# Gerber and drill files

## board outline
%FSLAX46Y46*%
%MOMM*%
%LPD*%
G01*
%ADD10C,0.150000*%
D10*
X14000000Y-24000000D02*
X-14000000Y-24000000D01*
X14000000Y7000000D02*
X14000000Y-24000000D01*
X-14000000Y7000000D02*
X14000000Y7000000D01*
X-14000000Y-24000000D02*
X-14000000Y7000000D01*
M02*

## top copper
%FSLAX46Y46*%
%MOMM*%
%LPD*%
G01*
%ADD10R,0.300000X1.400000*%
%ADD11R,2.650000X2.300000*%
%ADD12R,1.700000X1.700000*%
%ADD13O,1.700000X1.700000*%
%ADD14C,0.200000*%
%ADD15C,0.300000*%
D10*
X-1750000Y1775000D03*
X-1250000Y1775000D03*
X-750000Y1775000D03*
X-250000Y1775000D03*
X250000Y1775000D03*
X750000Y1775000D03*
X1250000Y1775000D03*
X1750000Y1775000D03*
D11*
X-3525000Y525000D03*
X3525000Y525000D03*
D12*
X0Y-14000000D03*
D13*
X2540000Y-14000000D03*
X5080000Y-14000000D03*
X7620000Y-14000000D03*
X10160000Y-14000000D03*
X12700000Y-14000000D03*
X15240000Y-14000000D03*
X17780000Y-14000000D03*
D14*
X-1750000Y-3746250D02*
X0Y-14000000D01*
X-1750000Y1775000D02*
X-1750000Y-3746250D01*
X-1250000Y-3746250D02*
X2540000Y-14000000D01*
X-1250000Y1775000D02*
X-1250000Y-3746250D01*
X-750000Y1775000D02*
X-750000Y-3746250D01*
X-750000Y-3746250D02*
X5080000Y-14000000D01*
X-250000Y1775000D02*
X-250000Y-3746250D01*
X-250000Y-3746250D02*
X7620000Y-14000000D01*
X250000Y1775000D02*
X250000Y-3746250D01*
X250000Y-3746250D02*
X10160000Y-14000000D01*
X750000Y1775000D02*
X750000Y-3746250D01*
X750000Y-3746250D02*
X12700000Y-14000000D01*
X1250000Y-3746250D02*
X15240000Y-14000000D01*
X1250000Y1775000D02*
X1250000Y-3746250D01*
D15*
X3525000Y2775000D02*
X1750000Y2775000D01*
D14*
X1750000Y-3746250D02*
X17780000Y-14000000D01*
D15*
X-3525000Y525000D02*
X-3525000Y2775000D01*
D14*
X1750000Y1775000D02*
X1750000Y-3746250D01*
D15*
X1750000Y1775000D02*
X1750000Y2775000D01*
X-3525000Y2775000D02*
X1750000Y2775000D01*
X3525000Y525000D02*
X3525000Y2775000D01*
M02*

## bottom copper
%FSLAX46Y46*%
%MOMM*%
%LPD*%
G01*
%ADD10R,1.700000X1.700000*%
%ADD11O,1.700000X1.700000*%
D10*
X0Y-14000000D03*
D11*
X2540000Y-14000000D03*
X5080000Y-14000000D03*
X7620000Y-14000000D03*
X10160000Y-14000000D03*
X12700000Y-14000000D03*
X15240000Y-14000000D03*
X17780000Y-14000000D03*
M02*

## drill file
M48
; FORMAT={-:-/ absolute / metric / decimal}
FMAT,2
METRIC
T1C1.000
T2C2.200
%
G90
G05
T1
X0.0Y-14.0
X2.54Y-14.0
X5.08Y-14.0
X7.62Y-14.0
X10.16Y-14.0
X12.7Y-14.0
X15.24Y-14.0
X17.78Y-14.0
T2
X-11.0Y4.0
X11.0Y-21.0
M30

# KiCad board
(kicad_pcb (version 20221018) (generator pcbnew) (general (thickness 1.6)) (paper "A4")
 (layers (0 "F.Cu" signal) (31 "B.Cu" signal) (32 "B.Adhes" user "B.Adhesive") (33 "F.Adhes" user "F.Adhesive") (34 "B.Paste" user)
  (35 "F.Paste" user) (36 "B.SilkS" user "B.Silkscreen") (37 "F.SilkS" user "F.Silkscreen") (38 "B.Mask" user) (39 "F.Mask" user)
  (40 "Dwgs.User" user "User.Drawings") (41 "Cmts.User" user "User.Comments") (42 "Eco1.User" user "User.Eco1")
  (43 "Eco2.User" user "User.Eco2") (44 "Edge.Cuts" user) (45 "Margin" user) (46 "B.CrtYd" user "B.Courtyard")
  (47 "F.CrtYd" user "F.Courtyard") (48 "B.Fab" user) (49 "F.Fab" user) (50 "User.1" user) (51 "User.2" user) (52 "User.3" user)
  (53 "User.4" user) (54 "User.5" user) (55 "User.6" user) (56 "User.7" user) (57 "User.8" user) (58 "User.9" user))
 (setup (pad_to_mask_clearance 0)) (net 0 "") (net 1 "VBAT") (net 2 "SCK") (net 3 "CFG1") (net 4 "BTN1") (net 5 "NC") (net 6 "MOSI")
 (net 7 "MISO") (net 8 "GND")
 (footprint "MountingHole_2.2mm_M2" (layer "F.Cu") (at -11 -4)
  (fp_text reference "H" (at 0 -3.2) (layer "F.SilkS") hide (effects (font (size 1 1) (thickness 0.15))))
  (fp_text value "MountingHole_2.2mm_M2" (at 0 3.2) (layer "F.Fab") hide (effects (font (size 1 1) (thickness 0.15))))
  (pad "" np_thru_hole circle (at 0 0) (size 2.2 2.2) (drill 2.2) (layers "*.Cu" "*.Mask")))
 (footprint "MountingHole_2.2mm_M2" (layer "F.Cu") (at 11 21)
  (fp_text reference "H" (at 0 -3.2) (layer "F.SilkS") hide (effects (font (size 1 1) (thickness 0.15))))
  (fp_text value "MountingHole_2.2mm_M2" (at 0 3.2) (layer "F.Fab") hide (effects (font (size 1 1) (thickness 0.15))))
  (pad "" np_thru_hole circle (at 0 0) (size 2.2 2.2) (drill 2.2) (layers "*.Cu" "*.Mask")))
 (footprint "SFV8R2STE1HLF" (layer "F.Cu") (at 0 0)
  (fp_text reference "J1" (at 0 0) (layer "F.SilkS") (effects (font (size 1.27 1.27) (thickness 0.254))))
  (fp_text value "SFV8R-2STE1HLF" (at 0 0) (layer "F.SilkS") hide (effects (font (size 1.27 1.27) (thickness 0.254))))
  (pad "1" smd rect (at -1.75 -1.775) (size 0.3 1.4) (layers "F.Cu" "F.Paste" "F.Mask") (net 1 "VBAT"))
  (pad "2" smd rect (at -1.25 -1.775) (size 0.3 1.4) (layers "F.Cu" "F.Paste" "F.Mask") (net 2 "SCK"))
  (pad "3" smd rect (at -0.75 -1.775) (size 0.3 1.4) (layers "F.Cu" "F.Paste" "F.Mask") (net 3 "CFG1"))
  (pad "4" smd rect (at -0.25 -1.775) (size 0.3 1.4) (layers "F.Cu" "F.Paste" "F.Mask") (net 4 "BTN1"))
  (pad "5" smd rect (at 0.25 -1.775) (size 0.3 1.4) (layers "F.Cu" "F.Paste" "F.Mask") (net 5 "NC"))
  (pad "6" smd rect (at 0.75 -1.775) (size 0.3 1.4) (layers "F.Cu" "F.Paste" "F.Mask") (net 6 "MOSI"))
  (pad "7" smd rect (at 1.25 -1.775) (size 0.3 1.4) (layers "F.Cu" "F.Paste" "F.Mask") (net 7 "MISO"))
  (pad "8" smd rect (at 1.75 -1.775) (size 0.3 1.4) (layers "F.Cu" "F.Paste" "F.Mask") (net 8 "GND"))
  (pad "M1" smd rect (at -3.525 -0.525 90) (size 2.3 2.65) (layers "F.Cu" "F.Paste" "F.Mask") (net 8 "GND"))
  (pad "M2" smd rect (at 3.525 -0.525 90) (size 2.3 2.65) (layers "F.Cu" "F.Paste" "F.Mask") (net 8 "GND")))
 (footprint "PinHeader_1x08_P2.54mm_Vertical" (layer "F.Cu") (at 0 14 90)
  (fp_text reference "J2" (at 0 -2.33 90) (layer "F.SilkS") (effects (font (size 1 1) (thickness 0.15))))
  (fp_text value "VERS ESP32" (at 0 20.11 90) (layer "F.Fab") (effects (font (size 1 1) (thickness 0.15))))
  (pad "1" thru_hole rect (at 0 0 90) (size 1.7 1.7) (drill 1) (layers "*.Cu" "*.Mask") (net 1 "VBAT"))
  (pad "2" thru_hole oval (at 0 2.54 90) (size 1.7 1.7) (drill 1) (layers "*.Cu" "*.Mask") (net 2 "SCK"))
  (pad "3" thru_hole oval (at 0 5.08 90) (size 1.7 1.7) (drill 1) (layers "*.Cu" "*.Mask") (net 3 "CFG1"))
  (pad "4" thru_hole oval (at 0 7.62 90) (size 1.7 1.7) (drill 1) (layers "*.Cu" "*.Mask") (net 4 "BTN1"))
  (pad "5" thru_hole oval (at 0 10.16 90) (size 1.7 1.7) (drill 1) (layers "*.Cu" "*.Mask") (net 5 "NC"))
  (pad "6" thru_hole oval (at 0 12.7 90) (size 1.7 1.7) (drill 1) (layers "*.Cu" "*.Mask") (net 6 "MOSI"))
  (pad "7" thru_hole oval (at 0 15.24 90) (size 1.7 1.7) (drill 1) (layers "*.Cu" "*.Mask") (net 7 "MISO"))
  (pad "8" thru_hole oval (at 0 17.78 90) (size 1.7 1.7) (drill 1) (layers "*.Cu" "*.Mask") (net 8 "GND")))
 (gr_line (start 14 24) (end -14 24) (stroke (width 0.15) (type default)) (layer "Edge.Cuts"))
 (gr_line (start 14 -7) (end 14 24) (stroke (width 0.15) (type default)) (layer "Edge.Cuts"))
 (gr_line (start -14 -7) (end 14 -7) (stroke (width 0.15) (type default)) (layer "Edge.Cuts"))
 (gr_line (start -14 24) (end -14 -7) (stroke (width 0.15) (type default)) (layer "Edge.Cuts"))
 (segment (start -1.75 3.74625) (end 0 14) (width 0.2) (layer "F.Cu") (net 1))
 (segment (start -1.75 -1.775) (end -1.75 3.74625) (width 0.2) (layer "F.Cu") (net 1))
 (segment (start -1.25 3.74625) (end 2.54 14) (width 0.2) (layer "F.Cu") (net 2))
 (segment (start -1.25 -1.775) (end -1.25 3.74625) (width 0.2) (layer "F.Cu") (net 2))
 (segment (start -0.75 -1.775) (end -0.75 3.74625) (width 0.2) (layer "F.Cu") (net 3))
 (segment (start -0.75 3.74625) (end 5.08 14) (width 0.2) (layer "F.Cu") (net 3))
 (segment (start -0.25 -1.775) (end -0.25 3.74625) (width 0.2) (layer "F.Cu") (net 4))
 (segment (start -0.25 3.74625) (end 7.62 14) (width 0.2) (layer "F.Cu") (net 4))
 (segment (start 0.25 -1.775) (end 0.25 3.74625) (width 0.2) (layer "F.Cu") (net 5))
 (segment (start 0.25 3.74625) (end 10.16 14) (width 0.2) (layer "F.Cu") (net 5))
 (segment (start 0.75 -1.775) (end 0.75 3.74625) (width 0.2) (layer "F.Cu") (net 6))
 (segment (start 0.75 3.74625) (end 12.7 14) (width 0.2) (layer "F.Cu") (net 6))
 (segment (start 1.25 3.74625) (end 15.24 14) (width 0.2) (layer "F.Cu") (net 7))
 (segment (start 1.25 -1.775) (end 1.25 3.74625) (width 0.2) (layer "F.Cu") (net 7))
 (segment (start 3.525 -2.775) (end 1.75 -2.775) (width 0.3) (layer "F.Cu") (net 8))
 (segment (start 1.75 3.74625) (end 17.78 14) (width 0.2) (layer "F.Cu") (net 8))
 (segment (start -3.525 -0.525) (end -3.525 -2.775) (width 0.3) (layer "F.Cu") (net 8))
 (segment (start 1.75 -1.775) (end 1.75 3.74625) (width 0.2) (layer "F.Cu") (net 8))
 (segment (start 1.75 -1.775) (end 1.75 -2.775) (width 0.3) (layer "F.Cu") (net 8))
 (segment (start -3.525 -2.775) (end 1.75 -2.775) (width 0.3) (layer "F.Cu") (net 8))
 (segment (start 3.525 -0.525) (end 3.525 -2.775) (width 0.3) (layer "F.Cu") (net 8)))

